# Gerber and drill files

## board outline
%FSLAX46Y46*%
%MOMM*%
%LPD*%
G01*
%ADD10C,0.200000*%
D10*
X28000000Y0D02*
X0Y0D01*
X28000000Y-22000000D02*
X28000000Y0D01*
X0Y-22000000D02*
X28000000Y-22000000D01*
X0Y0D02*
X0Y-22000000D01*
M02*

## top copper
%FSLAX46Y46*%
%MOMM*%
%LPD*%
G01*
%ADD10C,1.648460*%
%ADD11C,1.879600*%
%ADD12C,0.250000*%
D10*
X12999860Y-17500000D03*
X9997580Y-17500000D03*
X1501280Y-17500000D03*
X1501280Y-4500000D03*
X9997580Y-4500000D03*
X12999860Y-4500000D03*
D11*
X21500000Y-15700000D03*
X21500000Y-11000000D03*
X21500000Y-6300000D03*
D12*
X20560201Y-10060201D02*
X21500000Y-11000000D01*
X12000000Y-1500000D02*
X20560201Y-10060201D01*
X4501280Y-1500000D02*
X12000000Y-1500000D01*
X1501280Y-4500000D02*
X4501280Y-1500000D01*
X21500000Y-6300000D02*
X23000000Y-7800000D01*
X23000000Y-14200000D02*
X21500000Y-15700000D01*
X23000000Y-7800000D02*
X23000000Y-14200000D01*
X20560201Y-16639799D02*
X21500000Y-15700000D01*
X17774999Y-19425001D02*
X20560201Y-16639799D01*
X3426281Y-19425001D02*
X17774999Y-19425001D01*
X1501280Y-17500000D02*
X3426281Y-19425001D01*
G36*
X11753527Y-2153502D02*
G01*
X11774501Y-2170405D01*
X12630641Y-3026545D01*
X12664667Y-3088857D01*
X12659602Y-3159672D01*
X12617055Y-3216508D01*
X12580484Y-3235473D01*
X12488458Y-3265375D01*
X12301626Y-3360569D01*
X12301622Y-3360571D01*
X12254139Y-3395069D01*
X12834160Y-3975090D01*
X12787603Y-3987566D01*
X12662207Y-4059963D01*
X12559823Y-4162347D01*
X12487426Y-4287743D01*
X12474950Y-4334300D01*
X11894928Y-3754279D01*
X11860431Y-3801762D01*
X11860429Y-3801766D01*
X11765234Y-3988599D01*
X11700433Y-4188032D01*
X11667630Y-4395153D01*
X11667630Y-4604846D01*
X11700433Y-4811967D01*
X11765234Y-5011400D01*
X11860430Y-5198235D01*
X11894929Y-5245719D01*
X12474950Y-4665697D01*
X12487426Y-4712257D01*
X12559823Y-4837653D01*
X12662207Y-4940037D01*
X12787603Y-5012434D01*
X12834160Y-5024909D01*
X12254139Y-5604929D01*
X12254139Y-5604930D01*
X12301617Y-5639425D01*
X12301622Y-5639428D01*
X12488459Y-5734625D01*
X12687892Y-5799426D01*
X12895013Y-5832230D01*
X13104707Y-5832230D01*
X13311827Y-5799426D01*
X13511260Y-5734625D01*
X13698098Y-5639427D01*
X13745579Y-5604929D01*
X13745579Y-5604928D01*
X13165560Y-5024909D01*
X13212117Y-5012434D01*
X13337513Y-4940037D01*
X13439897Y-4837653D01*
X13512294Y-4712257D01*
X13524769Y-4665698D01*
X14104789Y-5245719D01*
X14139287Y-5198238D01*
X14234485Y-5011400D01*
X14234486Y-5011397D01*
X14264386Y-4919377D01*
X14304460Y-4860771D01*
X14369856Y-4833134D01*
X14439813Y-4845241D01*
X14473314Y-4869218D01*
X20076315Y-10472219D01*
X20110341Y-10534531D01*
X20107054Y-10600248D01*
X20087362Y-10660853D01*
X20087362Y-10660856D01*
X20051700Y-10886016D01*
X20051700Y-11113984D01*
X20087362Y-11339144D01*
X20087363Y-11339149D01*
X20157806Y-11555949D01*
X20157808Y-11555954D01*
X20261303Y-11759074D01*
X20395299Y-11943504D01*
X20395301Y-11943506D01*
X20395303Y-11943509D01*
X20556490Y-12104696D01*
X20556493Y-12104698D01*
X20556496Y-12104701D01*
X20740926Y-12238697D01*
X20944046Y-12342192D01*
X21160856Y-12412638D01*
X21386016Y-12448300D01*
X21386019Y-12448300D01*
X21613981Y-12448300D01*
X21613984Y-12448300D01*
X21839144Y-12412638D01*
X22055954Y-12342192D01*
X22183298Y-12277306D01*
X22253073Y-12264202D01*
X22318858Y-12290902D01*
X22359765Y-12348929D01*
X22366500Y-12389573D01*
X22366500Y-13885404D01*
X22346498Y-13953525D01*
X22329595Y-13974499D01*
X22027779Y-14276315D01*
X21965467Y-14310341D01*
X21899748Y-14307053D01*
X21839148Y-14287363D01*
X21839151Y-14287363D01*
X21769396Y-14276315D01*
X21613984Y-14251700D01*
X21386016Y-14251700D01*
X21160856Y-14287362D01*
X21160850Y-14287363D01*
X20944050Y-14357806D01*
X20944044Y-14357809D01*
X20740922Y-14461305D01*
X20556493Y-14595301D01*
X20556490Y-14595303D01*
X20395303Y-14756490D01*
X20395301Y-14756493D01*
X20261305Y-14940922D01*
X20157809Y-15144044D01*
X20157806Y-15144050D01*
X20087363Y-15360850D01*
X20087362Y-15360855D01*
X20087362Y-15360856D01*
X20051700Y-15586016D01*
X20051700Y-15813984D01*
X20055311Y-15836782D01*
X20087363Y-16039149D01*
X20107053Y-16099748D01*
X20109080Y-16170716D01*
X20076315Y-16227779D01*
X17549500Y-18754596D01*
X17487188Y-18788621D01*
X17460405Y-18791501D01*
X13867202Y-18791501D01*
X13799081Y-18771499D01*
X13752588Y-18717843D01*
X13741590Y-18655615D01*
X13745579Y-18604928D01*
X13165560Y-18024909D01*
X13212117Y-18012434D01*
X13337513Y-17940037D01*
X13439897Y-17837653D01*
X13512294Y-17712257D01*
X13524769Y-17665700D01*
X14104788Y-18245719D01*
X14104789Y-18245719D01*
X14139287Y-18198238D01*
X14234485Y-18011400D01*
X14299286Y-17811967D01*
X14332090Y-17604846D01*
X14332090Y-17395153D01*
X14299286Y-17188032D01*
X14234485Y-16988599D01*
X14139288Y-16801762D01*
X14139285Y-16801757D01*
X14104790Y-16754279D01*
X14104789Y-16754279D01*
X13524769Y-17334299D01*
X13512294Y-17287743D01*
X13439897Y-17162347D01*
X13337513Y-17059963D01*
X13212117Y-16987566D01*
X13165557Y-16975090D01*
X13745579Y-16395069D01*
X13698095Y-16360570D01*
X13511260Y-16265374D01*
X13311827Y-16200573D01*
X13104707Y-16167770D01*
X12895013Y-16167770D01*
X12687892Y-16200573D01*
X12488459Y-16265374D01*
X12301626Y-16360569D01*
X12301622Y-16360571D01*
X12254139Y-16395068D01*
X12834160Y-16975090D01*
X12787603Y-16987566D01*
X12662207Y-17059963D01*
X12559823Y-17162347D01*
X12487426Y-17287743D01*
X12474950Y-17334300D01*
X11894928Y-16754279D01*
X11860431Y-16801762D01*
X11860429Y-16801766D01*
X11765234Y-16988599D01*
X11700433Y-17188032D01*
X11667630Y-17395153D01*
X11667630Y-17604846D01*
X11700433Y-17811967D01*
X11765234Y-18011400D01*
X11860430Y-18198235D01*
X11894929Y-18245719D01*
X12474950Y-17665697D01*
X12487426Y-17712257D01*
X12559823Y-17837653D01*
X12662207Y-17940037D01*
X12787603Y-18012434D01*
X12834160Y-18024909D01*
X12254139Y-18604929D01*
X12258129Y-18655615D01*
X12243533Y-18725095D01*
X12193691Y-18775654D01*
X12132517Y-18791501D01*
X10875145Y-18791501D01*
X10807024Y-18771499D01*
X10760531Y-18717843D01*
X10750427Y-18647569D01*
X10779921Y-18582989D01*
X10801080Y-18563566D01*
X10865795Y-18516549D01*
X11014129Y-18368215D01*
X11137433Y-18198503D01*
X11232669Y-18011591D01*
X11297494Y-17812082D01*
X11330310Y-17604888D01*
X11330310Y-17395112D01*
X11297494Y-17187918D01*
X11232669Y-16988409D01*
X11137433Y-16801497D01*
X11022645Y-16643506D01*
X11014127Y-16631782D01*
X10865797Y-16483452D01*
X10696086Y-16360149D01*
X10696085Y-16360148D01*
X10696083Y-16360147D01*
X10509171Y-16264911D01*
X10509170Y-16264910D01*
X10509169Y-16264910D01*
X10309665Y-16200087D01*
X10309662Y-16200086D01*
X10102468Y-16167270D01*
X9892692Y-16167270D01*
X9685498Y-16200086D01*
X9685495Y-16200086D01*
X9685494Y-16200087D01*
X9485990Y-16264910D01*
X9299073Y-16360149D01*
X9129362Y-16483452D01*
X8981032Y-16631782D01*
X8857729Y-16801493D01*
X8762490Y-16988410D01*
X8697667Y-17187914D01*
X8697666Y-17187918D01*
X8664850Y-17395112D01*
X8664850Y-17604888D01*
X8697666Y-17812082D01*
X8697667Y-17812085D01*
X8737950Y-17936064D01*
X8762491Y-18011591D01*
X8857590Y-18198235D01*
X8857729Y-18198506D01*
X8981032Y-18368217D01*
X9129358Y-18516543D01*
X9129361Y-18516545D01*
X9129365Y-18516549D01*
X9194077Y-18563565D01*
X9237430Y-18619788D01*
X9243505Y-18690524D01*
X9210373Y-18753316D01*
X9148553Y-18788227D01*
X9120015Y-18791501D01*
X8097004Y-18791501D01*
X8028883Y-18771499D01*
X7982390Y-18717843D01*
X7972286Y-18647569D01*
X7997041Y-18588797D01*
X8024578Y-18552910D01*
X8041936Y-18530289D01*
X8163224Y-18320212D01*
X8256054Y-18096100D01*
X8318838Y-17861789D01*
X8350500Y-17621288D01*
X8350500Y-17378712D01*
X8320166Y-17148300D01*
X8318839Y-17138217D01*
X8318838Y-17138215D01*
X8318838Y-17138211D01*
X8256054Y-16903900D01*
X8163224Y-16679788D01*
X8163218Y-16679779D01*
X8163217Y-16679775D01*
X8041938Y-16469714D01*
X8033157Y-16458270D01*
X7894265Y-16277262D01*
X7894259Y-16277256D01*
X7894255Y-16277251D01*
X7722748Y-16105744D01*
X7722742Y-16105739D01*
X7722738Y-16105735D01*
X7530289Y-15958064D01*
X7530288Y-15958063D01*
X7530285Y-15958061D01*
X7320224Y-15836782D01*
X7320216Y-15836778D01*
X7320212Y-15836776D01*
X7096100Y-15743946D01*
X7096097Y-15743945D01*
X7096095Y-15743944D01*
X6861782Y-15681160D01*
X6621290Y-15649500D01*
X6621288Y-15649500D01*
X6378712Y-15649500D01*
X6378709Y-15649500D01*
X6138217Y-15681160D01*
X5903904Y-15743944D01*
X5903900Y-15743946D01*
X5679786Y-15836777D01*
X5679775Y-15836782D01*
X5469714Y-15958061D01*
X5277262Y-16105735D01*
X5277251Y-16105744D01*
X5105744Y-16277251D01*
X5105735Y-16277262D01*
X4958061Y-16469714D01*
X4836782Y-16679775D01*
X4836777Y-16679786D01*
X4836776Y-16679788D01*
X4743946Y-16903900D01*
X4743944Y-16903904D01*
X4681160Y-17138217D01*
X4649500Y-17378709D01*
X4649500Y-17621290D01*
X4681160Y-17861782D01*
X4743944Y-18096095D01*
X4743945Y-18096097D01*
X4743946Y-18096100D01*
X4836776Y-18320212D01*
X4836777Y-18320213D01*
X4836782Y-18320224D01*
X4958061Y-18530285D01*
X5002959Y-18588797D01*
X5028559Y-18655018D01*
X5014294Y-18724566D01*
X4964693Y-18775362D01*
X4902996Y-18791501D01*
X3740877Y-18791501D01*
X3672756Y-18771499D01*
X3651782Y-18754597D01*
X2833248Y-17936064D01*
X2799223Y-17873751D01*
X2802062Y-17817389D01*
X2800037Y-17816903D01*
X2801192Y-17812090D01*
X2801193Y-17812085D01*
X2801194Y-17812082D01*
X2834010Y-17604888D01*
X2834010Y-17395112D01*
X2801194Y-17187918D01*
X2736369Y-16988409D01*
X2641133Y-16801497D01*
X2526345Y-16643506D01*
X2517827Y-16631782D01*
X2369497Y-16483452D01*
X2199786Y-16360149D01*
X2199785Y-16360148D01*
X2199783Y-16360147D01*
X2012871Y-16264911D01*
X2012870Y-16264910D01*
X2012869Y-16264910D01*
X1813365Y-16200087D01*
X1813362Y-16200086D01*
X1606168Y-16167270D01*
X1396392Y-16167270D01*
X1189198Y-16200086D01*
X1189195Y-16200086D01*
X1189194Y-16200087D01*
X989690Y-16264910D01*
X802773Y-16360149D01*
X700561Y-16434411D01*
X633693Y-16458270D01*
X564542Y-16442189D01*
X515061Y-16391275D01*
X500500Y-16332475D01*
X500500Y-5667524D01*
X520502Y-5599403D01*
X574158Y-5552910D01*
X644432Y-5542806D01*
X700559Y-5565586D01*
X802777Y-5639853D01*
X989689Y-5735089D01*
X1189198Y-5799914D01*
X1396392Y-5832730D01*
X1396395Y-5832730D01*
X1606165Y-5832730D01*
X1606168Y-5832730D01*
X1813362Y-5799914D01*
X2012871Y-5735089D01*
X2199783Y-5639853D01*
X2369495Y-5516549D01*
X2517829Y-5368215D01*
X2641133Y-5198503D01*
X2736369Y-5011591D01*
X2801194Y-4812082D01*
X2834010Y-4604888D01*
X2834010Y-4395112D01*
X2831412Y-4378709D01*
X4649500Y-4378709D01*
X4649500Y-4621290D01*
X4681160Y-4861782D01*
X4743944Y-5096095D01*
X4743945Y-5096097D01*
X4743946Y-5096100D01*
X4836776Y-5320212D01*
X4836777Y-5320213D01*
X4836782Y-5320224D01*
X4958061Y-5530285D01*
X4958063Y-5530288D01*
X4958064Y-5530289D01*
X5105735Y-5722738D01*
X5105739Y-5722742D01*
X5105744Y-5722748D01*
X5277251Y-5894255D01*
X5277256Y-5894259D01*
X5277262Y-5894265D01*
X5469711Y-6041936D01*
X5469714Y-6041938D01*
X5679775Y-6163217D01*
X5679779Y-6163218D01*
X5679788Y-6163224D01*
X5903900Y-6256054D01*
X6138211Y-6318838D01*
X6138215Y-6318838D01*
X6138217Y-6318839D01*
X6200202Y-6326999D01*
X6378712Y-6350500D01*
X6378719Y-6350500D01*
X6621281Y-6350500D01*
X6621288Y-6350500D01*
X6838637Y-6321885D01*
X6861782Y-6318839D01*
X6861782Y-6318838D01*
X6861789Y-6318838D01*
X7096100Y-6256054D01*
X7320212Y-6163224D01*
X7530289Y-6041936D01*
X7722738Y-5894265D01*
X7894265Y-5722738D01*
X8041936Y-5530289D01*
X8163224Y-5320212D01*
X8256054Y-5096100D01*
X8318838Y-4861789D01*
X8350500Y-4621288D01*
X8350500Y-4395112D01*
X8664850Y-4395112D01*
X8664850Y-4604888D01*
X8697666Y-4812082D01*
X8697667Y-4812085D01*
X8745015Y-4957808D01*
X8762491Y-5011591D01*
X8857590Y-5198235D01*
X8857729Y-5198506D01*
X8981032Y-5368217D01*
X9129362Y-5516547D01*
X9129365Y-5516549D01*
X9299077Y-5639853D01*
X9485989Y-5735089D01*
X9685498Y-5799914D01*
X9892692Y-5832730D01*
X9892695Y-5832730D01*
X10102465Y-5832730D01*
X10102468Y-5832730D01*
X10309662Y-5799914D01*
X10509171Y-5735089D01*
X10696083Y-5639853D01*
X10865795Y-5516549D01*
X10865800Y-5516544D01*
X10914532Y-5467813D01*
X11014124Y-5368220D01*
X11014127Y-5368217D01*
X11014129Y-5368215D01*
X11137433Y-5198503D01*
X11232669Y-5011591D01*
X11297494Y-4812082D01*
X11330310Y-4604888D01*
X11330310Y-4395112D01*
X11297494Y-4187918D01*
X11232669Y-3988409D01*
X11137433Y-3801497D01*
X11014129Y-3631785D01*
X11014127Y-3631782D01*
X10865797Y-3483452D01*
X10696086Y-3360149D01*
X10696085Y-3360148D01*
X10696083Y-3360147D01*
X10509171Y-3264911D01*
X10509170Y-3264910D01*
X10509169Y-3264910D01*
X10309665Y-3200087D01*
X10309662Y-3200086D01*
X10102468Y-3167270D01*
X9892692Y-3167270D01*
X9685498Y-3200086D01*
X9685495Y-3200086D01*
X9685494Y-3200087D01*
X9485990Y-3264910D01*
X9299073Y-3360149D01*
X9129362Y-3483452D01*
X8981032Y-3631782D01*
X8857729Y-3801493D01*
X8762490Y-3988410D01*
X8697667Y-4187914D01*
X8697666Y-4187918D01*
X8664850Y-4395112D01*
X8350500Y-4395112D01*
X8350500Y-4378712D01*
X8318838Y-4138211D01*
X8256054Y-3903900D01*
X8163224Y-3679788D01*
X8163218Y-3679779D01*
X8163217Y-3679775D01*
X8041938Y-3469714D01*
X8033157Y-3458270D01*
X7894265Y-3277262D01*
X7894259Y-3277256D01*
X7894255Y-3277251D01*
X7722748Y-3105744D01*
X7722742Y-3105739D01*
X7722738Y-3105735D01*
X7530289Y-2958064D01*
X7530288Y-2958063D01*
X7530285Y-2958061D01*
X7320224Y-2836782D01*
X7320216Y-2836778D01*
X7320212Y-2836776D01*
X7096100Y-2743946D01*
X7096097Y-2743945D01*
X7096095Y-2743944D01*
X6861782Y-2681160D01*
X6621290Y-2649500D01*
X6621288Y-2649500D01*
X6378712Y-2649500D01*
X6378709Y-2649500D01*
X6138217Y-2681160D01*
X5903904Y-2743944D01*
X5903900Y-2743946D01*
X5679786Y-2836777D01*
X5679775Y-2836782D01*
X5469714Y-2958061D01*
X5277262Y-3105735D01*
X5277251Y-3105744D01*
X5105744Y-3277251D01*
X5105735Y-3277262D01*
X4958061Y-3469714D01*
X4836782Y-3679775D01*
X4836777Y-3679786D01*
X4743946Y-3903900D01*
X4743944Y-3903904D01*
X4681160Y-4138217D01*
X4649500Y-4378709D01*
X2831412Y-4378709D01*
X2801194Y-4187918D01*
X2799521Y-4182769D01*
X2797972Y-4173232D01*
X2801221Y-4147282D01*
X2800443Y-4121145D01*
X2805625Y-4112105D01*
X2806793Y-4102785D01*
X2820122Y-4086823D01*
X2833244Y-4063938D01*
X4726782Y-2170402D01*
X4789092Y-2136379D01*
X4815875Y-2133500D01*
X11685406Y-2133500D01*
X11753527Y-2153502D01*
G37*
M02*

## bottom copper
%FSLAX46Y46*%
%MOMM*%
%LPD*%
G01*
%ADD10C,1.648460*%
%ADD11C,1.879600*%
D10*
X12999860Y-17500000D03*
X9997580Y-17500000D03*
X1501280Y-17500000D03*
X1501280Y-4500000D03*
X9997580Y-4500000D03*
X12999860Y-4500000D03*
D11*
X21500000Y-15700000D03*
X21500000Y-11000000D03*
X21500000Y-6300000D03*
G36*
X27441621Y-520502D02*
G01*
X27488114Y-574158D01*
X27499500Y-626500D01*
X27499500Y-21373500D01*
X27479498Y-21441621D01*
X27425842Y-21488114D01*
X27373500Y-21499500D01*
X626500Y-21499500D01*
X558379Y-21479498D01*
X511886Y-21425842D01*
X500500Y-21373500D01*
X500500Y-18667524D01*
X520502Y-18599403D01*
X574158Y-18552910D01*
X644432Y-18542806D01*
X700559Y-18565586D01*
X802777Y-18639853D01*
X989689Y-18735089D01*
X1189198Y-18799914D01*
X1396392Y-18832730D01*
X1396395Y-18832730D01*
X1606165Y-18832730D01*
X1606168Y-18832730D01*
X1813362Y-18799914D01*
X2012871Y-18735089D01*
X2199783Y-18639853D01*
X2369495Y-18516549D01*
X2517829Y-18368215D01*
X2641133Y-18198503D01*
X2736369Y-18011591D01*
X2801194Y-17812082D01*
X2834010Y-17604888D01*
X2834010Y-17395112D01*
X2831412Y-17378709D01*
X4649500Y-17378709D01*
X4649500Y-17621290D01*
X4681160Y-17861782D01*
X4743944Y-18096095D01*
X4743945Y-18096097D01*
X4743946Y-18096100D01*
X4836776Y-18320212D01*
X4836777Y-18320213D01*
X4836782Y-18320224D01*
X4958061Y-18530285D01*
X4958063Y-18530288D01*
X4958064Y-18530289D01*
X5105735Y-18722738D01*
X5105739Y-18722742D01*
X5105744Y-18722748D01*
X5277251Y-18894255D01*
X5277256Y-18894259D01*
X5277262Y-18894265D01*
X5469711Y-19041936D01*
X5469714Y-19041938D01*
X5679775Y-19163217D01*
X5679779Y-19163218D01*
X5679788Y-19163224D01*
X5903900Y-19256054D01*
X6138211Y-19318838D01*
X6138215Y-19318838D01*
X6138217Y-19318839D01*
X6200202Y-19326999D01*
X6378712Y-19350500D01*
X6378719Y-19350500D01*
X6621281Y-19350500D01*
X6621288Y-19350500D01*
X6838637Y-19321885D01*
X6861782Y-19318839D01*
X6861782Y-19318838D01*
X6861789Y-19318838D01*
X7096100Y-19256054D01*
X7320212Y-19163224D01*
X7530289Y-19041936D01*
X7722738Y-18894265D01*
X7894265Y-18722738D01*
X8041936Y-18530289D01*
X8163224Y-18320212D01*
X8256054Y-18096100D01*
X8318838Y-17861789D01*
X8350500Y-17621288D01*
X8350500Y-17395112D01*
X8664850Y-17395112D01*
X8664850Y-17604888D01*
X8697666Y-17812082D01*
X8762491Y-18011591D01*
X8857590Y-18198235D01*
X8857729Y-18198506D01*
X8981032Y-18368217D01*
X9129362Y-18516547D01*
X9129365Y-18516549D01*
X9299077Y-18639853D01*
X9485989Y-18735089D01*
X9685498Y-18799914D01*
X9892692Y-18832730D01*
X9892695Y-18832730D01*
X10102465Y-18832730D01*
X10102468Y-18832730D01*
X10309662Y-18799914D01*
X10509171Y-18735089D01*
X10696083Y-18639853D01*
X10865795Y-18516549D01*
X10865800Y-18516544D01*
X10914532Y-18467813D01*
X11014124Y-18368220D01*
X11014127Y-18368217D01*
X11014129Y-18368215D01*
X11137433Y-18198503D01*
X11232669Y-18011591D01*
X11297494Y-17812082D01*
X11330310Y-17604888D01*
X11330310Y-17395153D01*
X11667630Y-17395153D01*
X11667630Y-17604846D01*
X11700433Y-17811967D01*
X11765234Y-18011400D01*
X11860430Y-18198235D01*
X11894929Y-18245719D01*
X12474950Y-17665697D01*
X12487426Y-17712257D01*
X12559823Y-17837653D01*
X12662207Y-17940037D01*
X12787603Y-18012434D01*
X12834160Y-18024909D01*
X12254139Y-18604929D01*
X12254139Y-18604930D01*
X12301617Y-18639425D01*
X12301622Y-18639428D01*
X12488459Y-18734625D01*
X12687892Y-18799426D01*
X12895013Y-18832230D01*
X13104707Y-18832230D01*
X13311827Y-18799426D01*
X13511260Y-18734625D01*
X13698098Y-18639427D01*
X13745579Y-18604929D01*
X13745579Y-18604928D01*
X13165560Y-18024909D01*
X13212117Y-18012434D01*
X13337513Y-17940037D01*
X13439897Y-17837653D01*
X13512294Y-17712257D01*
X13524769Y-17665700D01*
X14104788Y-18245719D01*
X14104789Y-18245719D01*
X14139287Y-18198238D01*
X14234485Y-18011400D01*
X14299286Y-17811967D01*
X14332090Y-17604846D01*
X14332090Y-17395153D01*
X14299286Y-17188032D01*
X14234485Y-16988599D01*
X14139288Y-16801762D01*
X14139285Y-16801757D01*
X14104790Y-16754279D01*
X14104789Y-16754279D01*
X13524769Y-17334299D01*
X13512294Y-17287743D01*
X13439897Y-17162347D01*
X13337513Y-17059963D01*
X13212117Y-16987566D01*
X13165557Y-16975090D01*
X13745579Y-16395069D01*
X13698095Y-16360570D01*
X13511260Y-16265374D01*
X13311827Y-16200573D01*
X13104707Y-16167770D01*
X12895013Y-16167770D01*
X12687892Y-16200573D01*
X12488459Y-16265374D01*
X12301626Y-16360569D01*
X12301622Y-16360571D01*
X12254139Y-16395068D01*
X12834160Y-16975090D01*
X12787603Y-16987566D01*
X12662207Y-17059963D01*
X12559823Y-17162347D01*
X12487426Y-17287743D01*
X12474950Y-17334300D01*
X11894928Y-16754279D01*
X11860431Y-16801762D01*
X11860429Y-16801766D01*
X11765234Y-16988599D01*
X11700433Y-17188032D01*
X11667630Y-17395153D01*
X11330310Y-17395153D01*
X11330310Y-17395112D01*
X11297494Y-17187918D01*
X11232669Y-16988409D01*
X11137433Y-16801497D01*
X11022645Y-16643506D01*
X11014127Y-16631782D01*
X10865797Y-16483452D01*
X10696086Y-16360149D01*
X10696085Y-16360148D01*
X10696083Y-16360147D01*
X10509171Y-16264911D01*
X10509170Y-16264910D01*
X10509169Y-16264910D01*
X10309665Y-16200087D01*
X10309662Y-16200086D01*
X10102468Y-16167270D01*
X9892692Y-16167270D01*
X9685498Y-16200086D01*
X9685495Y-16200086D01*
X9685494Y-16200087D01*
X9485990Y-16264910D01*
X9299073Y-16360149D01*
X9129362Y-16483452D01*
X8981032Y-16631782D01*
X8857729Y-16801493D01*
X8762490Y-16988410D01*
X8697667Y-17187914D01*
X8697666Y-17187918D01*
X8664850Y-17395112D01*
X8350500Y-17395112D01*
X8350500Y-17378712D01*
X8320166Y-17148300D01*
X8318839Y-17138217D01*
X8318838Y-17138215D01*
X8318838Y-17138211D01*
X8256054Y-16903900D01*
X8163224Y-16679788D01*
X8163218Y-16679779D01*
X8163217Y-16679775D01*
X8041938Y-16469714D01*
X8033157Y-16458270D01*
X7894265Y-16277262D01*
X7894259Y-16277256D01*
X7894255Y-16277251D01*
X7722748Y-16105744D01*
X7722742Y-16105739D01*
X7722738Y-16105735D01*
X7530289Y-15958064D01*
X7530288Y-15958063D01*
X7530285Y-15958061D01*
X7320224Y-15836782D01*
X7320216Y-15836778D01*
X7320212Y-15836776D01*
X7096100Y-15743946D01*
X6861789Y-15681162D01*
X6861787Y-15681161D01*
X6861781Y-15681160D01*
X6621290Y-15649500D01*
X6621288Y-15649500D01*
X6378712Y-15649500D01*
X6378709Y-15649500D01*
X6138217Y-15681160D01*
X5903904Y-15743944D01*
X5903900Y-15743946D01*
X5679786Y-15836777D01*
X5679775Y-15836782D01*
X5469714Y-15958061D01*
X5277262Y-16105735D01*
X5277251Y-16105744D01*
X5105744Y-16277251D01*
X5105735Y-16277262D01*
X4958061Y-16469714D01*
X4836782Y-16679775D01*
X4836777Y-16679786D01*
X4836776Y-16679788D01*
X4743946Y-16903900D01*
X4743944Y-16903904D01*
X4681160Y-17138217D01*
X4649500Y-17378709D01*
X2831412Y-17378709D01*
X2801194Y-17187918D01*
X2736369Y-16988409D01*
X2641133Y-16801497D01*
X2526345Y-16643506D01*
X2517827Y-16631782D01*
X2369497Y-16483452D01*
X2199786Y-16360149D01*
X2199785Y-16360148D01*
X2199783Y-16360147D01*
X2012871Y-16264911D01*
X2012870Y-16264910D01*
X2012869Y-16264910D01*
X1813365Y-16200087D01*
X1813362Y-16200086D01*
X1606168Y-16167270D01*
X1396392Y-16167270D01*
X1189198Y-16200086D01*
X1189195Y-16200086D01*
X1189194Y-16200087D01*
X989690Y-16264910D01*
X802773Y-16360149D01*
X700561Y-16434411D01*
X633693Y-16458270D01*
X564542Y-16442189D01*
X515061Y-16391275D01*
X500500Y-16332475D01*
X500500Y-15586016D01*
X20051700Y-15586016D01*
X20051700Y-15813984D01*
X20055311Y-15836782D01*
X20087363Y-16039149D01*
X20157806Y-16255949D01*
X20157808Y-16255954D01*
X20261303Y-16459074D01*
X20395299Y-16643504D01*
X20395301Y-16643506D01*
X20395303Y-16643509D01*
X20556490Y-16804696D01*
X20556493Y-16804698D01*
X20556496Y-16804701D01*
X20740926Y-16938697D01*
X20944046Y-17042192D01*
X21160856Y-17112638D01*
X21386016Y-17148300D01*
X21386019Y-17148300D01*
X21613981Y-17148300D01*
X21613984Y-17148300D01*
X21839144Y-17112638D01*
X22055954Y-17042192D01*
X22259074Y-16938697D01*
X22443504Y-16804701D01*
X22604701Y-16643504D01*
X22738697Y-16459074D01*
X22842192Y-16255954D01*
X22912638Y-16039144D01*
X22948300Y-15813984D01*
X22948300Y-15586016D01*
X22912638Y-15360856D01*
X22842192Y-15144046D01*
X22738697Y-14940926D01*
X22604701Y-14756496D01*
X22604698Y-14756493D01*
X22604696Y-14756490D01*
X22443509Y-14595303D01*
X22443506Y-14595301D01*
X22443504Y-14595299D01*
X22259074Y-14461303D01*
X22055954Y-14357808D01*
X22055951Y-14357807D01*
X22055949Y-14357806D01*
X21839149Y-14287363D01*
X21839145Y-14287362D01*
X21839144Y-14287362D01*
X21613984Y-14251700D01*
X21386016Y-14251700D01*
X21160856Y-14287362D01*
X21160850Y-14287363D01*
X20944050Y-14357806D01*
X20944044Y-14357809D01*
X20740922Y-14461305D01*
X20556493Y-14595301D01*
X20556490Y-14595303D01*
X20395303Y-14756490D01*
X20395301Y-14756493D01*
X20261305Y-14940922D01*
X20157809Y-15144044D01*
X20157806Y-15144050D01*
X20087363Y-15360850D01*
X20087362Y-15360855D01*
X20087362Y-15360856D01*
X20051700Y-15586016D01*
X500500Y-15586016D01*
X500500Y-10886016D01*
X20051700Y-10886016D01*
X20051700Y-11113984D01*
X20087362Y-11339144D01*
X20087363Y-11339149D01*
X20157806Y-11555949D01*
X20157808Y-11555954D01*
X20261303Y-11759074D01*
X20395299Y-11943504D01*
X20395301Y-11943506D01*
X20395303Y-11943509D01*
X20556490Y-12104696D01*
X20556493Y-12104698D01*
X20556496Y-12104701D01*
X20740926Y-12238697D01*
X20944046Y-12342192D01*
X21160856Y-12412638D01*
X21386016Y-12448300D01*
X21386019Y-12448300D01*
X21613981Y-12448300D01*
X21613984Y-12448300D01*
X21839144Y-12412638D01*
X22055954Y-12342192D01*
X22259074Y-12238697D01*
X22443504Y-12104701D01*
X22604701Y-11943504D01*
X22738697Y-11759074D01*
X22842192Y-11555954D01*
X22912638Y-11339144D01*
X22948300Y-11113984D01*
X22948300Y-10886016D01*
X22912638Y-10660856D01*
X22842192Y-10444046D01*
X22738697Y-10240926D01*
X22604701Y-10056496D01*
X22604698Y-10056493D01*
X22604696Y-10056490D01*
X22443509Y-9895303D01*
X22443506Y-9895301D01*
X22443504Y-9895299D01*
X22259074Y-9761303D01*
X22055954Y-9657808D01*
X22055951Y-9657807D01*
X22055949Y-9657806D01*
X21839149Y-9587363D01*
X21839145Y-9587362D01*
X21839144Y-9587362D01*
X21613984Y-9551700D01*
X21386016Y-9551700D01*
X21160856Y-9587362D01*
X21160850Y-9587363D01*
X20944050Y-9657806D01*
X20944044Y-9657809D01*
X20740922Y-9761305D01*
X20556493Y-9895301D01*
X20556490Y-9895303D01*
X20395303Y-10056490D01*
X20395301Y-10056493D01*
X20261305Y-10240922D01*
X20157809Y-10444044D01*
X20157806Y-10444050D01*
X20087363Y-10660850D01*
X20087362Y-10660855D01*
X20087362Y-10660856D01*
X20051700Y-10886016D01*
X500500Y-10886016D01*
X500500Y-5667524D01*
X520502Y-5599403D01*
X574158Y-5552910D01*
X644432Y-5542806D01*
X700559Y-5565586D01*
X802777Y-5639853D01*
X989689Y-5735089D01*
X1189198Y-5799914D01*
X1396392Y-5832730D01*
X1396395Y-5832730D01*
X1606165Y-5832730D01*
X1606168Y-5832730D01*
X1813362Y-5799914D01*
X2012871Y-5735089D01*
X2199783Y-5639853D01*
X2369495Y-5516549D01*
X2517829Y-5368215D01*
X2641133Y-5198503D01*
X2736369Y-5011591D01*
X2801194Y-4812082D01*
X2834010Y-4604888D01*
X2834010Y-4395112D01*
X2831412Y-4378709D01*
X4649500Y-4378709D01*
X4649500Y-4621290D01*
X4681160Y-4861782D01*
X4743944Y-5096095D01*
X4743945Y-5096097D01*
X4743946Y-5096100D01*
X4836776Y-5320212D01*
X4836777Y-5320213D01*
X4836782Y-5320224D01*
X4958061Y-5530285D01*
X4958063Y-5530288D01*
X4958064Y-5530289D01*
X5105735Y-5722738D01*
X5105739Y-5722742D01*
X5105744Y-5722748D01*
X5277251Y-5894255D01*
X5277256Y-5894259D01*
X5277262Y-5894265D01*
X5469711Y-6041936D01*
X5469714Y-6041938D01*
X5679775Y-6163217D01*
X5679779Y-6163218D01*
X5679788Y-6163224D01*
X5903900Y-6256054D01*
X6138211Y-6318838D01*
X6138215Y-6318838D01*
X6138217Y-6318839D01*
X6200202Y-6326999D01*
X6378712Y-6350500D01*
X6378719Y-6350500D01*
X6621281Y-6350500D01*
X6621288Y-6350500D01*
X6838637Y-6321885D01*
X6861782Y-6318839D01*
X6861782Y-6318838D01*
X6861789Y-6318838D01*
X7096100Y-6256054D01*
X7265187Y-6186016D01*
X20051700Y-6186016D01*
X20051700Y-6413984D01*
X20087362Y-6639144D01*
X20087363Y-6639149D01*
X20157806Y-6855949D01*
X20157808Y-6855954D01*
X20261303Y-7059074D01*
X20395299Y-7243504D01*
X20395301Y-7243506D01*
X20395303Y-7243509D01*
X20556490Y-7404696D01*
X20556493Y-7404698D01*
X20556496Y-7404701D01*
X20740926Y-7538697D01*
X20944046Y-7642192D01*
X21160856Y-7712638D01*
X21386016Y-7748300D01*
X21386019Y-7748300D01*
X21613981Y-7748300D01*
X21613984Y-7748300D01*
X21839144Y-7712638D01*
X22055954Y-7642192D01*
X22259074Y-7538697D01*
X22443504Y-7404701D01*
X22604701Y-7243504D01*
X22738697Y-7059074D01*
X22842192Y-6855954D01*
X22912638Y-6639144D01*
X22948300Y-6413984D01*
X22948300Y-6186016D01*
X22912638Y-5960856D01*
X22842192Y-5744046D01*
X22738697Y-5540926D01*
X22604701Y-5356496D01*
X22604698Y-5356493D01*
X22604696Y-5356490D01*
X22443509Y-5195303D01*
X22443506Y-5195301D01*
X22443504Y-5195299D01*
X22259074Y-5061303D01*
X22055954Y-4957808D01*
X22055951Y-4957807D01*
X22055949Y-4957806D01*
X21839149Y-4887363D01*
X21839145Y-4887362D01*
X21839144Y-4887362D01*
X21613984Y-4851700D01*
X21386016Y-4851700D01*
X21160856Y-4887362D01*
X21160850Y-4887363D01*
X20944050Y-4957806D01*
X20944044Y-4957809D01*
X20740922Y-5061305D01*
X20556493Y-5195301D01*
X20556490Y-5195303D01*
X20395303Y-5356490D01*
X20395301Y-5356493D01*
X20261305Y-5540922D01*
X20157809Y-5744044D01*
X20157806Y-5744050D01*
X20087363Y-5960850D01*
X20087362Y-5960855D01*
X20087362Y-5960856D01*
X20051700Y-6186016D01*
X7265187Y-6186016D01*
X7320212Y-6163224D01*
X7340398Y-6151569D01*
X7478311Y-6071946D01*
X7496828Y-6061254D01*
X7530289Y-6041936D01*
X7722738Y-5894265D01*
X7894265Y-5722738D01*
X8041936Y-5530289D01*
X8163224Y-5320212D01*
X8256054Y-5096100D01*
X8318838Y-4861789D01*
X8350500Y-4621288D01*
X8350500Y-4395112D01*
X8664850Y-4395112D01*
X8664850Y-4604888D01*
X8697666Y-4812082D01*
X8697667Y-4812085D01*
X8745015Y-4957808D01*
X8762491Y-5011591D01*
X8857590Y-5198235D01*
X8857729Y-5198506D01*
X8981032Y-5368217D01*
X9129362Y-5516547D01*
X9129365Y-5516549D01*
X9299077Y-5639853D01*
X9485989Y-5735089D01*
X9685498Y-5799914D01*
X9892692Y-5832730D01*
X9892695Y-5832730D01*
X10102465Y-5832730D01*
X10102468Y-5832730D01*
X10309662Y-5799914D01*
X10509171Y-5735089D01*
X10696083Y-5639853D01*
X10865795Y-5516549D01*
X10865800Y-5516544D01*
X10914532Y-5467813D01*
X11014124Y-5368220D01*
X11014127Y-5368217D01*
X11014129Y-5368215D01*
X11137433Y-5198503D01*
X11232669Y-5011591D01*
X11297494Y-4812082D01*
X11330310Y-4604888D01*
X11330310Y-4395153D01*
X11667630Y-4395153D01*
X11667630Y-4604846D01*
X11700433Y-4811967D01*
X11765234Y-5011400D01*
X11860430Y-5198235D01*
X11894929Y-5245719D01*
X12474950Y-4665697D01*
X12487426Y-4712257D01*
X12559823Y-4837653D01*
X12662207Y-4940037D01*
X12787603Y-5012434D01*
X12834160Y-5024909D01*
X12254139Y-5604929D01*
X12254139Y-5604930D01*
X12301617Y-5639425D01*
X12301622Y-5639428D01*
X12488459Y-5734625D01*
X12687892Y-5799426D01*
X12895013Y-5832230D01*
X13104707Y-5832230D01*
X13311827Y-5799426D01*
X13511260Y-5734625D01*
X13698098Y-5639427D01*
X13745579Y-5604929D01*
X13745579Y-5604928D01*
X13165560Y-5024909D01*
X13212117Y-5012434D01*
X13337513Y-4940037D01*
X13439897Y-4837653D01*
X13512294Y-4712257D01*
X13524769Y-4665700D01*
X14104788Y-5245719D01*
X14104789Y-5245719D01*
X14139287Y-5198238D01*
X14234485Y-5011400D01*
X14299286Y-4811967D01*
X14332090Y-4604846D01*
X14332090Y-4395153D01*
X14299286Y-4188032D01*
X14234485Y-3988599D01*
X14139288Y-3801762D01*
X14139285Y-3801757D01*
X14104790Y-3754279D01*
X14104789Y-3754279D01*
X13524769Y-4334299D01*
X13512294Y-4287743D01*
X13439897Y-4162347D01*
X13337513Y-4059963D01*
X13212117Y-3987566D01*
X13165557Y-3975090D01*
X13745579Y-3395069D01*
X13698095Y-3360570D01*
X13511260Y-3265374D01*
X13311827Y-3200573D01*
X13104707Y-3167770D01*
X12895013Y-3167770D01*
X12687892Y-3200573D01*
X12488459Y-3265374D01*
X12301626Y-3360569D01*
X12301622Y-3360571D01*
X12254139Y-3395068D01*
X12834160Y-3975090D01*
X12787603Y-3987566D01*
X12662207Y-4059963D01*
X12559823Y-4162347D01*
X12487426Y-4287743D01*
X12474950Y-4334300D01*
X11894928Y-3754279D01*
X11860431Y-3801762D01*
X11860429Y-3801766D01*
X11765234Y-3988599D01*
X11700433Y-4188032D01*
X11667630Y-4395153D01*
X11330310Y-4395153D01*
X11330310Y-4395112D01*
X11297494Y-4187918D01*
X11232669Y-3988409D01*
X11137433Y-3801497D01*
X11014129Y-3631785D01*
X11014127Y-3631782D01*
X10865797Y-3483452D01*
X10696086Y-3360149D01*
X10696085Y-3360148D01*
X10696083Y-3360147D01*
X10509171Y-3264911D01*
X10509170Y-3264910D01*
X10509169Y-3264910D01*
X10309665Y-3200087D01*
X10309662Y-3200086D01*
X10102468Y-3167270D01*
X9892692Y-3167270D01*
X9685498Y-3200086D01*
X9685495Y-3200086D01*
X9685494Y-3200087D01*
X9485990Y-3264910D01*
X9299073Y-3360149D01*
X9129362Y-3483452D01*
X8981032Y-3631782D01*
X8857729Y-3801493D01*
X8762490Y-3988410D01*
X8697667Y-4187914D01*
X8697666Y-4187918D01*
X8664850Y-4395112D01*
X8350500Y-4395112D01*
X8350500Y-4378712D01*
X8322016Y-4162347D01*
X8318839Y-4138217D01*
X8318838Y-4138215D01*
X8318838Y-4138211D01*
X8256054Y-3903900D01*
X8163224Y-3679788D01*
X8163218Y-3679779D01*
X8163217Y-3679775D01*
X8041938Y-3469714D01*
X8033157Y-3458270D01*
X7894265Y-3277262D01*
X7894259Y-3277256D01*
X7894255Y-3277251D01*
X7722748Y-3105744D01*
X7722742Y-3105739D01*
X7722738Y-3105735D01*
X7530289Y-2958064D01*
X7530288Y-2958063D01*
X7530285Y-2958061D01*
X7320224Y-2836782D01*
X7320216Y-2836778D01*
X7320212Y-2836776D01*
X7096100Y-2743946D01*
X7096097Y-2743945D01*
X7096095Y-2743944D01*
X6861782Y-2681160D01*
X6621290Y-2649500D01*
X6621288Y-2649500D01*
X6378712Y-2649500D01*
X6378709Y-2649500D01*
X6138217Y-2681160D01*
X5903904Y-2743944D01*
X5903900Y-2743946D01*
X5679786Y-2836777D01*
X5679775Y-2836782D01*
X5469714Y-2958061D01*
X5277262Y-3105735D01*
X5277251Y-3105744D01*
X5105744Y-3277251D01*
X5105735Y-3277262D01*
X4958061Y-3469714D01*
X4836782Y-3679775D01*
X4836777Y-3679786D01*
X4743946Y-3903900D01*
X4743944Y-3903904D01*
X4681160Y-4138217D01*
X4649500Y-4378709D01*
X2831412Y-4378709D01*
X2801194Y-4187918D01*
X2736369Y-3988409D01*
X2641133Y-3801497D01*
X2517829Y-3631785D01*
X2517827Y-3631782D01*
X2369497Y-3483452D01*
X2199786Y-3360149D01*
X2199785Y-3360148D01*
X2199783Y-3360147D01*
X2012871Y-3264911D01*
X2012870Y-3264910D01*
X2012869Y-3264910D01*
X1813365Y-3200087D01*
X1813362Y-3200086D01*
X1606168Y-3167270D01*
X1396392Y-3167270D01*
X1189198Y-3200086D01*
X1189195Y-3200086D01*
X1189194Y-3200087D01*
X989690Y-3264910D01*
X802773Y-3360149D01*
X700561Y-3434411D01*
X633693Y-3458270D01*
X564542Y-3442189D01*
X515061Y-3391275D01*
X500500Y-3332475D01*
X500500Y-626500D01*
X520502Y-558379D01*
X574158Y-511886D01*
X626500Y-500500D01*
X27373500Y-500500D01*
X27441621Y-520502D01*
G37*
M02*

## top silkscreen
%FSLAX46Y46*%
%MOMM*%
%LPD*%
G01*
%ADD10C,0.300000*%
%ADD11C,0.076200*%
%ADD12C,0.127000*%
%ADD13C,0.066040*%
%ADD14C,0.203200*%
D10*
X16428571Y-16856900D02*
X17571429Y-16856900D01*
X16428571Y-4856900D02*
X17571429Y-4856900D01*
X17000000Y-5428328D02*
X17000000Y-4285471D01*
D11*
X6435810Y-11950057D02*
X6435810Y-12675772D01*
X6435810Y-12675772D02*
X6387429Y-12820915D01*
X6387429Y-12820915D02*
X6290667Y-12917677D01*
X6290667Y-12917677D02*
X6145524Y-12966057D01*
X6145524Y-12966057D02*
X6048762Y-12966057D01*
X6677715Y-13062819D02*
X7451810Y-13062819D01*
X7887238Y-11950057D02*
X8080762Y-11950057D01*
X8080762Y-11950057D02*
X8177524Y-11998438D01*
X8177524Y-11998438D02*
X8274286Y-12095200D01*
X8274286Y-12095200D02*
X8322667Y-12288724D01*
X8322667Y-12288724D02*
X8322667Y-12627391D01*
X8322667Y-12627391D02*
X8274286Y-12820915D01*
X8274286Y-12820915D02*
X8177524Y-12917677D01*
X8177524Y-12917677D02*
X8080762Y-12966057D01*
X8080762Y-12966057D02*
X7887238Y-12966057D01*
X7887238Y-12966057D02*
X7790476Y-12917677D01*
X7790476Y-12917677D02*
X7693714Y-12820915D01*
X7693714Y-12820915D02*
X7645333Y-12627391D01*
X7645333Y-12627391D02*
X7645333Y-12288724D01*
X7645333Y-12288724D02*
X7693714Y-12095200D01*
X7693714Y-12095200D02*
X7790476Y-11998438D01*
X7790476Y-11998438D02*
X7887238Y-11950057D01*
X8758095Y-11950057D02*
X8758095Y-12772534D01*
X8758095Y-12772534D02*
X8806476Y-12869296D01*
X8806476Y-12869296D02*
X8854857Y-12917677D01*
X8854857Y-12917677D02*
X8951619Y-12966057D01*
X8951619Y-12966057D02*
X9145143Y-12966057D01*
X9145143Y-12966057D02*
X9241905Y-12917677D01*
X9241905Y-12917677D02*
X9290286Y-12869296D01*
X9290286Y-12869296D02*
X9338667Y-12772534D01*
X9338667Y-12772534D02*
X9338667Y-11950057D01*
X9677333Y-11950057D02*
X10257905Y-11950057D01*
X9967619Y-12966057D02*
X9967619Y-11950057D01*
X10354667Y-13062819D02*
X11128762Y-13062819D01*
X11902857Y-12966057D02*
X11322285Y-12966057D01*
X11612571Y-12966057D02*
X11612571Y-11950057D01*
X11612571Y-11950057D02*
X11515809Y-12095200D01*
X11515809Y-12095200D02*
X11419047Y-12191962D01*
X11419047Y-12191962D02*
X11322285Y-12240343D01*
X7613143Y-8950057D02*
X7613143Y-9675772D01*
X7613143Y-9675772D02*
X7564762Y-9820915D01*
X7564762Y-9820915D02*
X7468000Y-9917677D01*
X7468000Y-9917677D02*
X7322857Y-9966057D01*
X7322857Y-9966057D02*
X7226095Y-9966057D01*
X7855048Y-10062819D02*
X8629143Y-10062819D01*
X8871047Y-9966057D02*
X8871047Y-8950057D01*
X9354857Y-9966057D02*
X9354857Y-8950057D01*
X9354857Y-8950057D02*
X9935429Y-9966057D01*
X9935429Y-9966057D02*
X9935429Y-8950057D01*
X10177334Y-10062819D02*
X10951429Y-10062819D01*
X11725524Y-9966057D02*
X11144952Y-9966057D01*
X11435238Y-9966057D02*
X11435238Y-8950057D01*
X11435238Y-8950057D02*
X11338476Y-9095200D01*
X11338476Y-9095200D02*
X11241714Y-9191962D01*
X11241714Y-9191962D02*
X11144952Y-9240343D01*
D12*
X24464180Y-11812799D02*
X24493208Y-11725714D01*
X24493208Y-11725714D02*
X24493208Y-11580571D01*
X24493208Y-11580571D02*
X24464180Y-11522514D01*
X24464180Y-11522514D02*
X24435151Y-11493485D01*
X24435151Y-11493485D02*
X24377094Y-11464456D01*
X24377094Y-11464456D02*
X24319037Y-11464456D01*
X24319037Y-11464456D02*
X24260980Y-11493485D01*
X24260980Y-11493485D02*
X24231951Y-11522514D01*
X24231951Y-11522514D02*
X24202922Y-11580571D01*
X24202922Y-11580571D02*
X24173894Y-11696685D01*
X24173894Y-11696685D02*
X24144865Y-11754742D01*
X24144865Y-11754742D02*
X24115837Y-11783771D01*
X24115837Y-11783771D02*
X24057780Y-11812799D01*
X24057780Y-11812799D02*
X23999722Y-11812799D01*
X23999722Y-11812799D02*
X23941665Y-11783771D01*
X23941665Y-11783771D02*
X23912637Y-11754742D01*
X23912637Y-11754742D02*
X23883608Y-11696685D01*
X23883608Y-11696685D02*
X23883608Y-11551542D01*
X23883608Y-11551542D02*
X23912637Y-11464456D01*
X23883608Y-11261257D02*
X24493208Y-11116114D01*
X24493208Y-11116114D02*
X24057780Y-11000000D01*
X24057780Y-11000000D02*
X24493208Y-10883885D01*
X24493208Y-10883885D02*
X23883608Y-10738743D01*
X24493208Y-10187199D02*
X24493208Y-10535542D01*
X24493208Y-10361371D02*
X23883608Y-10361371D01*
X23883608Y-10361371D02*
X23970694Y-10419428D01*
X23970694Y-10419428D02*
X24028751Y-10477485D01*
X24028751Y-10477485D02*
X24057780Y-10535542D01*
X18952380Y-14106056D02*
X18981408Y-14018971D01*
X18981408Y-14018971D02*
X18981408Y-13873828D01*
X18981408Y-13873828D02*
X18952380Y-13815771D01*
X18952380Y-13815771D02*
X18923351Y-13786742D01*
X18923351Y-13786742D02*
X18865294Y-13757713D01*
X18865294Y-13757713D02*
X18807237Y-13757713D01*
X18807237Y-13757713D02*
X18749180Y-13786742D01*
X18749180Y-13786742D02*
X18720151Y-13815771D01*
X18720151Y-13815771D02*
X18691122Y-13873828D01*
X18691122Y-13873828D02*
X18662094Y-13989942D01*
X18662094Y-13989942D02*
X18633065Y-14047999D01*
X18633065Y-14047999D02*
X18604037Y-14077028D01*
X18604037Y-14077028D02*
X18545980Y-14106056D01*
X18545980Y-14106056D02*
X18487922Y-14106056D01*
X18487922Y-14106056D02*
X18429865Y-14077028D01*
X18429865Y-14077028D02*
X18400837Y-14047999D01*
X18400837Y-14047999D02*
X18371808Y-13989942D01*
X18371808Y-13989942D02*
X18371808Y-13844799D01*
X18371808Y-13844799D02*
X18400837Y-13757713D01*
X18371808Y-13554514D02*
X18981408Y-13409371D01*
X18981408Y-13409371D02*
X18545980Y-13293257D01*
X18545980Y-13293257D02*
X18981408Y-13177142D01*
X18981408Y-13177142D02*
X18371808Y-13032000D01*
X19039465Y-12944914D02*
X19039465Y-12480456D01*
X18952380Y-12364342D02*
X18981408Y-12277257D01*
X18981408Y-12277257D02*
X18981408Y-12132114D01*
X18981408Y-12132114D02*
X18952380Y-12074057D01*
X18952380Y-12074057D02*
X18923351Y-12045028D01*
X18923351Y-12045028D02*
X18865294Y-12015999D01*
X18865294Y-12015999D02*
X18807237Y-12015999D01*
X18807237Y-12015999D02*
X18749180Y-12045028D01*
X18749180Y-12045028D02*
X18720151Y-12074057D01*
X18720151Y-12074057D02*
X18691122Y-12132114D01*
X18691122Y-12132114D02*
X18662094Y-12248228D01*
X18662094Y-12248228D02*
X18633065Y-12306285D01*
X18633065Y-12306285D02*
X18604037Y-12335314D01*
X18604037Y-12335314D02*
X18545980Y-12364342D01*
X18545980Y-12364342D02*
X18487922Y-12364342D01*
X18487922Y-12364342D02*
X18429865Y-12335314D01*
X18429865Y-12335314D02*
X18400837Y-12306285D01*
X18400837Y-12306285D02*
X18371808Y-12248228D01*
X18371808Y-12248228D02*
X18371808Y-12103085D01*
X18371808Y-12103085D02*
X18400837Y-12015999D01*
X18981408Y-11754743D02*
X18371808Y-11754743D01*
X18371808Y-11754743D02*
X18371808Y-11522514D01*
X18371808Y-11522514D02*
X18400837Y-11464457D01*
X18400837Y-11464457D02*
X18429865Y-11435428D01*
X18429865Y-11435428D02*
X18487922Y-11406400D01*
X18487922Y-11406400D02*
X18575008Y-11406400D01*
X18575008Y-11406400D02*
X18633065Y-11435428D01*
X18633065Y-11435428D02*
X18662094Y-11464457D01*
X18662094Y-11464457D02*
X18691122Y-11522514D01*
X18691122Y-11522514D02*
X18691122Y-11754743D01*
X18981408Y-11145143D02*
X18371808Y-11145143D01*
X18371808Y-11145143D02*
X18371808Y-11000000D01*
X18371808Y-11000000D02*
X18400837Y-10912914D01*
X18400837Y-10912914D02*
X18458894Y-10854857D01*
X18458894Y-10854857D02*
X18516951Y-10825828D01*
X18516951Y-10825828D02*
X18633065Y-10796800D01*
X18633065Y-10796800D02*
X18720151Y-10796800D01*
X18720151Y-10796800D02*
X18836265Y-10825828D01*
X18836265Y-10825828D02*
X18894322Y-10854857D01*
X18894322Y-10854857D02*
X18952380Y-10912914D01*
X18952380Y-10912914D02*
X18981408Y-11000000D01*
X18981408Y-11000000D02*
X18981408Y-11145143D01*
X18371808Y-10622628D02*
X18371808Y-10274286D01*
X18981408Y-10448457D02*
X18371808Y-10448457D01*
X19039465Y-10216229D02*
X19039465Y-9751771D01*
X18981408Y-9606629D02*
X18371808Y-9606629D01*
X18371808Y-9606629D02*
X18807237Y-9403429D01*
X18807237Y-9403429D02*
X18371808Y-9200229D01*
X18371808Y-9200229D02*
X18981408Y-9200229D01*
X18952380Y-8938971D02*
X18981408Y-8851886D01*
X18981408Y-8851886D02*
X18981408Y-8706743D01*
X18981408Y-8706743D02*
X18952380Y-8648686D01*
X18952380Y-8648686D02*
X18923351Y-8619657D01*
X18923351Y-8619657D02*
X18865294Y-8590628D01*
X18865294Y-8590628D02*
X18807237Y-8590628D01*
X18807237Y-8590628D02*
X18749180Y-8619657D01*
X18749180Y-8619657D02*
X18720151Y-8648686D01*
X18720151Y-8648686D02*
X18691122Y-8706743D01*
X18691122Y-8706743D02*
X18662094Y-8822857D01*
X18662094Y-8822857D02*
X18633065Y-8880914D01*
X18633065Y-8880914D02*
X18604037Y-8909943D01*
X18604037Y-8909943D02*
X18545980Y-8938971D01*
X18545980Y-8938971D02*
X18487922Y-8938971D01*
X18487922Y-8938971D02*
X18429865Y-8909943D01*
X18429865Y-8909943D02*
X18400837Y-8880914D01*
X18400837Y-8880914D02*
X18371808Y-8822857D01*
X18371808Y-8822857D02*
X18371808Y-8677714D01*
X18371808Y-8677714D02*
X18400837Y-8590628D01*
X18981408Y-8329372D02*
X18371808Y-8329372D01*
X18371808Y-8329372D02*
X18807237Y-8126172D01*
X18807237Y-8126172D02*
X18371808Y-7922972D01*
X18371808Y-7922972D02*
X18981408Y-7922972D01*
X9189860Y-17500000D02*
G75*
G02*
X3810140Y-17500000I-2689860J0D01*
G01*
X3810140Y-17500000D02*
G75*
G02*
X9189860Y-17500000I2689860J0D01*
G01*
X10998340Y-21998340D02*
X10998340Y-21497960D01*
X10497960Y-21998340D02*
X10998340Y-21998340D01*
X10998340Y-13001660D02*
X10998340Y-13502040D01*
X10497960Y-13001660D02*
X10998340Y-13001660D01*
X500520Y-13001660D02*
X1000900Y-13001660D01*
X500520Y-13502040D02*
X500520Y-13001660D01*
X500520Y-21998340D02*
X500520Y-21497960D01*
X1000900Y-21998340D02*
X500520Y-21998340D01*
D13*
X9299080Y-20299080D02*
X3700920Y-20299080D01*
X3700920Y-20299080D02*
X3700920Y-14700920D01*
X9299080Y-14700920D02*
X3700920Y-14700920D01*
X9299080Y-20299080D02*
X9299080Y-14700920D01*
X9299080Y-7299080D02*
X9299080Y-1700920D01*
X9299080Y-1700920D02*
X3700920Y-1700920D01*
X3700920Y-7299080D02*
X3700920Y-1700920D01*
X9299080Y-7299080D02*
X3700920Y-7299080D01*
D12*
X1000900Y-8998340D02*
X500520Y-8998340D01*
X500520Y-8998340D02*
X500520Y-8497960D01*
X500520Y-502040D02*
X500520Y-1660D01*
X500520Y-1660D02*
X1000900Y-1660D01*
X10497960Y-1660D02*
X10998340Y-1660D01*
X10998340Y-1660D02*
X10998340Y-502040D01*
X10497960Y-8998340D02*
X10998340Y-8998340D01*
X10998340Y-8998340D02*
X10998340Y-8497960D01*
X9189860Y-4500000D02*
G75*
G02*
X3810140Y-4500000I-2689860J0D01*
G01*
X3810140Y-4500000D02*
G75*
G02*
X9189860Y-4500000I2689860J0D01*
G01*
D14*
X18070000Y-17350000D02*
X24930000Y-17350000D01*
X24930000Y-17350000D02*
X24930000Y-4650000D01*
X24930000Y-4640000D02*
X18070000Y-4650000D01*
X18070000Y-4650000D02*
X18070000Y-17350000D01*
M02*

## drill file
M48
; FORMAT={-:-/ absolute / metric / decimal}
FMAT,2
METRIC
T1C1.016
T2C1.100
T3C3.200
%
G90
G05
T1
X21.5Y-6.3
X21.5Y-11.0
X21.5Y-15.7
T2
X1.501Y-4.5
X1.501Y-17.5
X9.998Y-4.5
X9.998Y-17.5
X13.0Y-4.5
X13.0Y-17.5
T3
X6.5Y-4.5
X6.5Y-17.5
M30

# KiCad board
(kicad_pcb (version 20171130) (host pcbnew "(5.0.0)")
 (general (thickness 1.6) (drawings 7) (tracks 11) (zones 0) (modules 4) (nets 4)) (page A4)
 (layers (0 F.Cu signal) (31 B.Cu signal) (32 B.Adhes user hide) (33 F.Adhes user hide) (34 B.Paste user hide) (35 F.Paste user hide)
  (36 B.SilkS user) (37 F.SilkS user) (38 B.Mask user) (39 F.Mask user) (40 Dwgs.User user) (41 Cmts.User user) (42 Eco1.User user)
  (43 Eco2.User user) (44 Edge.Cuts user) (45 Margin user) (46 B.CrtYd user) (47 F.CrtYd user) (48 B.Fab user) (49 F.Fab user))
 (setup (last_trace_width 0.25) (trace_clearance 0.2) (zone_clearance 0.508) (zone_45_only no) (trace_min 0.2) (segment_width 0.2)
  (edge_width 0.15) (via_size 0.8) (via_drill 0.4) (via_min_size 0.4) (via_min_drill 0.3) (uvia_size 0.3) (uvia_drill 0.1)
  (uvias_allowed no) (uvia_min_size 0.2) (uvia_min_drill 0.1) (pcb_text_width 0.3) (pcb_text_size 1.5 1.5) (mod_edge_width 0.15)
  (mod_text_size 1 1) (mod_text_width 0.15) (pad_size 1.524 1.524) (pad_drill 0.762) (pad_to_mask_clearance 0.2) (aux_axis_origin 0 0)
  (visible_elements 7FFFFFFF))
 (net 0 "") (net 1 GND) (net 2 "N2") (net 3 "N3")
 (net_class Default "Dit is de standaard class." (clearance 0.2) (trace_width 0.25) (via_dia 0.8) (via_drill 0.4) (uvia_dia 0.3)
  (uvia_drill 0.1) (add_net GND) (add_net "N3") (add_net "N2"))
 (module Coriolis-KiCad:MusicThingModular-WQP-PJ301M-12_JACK (layer F.Cu) (at 6.5 17.5 90)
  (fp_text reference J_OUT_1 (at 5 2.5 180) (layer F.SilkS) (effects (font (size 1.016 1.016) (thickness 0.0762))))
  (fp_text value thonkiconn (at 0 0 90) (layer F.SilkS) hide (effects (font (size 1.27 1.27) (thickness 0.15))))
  (fp_circle (center 0 0) (end 0 -2.68986) (layer F.SilkS) (width 0.127))
  (fp_line (start -4.49834 4.49834) (end -3.99796 4.49834) (layer F.SilkS) (width 0.127))
  (fp_line (start -4.49834 3.99796) (end -4.49834 4.49834) (layer F.SilkS) (width 0.127))
  (fp_line (start 4.49834 4.49834) (end 3.99796 4.49834) (layer F.SilkS) (width 0.127))
  (fp_line (start 4.49834 3.99796) (end 4.49834 4.49834) (layer F.SilkS) (width 0.127))
  (fp_line (start 4.49834 -5.99948) (end 4.49834 -5.4991) (layer F.SilkS) (width 0.127))
  (fp_line (start 3.99796 -5.99948) (end 4.49834 -5.99948) (layer F.SilkS) (width 0.127))
  (fp_line (start -4.49834 -5.99948) (end -3.99796 -5.99948) (layer F.SilkS) (width 0.127))
  (fp_line (start -4.49834 -5.4991) (end -4.49834 -5.99948) (layer F.SilkS) (width 0.127))
  (fp_line (start -2.79908 2.79908) (end -2.79908 -2.79908) (layer F.SilkS) (width 0.06604))
  (fp_line (start -2.79908 -2.79908) (end 2.79908 -2.79908) (layer F.SilkS) (width 0.06604))
  (fp_line (start 2.79908 2.79908) (end 2.79908 -2.79908) (layer F.SilkS) (width 0.06604))
  (fp_line (start -2.79908 2.79908) (end 2.79908 2.79908) (layer F.SilkS) (width 0.06604))
  (pad "" np_thru_hole circle (at 0 0 90) (size 3.2 3.2) (drill 3.2) (layers *.Cu *.Mask))
  (pad P$3_SLEEVE thru_hole circle (at 0 6.49986 90) (size 1.64846 1.64846) (drill 1.09982) (layers *.Cu *.Paste *.Mask) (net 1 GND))
  (pad P$2_SWITCH thru_hole circle (at 0 3.49758 90) (size 1.64846 1.64846) (drill 1.09982) (layers *.Cu *.Paste *.Mask))
  (pad P$1_TIP thru_hole circle (at 0 -4.99872 90) (size 1.64846 1.64846) (drill 1.09982) (layers *.Cu *.Paste *.Mask) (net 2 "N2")))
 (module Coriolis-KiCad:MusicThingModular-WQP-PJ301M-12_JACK (layer F.Cu) (at 6.5 4.5 90)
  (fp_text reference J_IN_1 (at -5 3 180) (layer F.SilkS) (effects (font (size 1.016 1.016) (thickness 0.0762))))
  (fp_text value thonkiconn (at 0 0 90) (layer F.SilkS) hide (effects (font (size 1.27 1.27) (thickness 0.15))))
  (fp_line (start -2.79908 2.79908) (end 2.79908 2.79908) (layer F.SilkS) (width 0.06604))
  (fp_line (start 2.79908 2.79908) (end 2.79908 -2.79908) (layer F.SilkS) (width 0.06604))
  (fp_line (start -2.79908 -2.79908) (end 2.79908 -2.79908) (layer F.SilkS) (width 0.06604))
  (fp_line (start -2.79908 2.79908) (end -2.79908 -2.79908) (layer F.SilkS) (width 0.06604))
  (fp_line (start -4.49834 -5.4991) (end -4.49834 -5.99948) (layer F.SilkS) (width 0.127))
  (fp_line (start -4.49834 -5.99948) (end -3.99796 -5.99948) (layer F.SilkS) (width 0.127))
  (fp_line (start 3.99796 -5.99948) (end 4.49834 -5.99948) (layer F.SilkS) (width 0.127))
  (fp_line (start 4.49834 -5.99948) (end 4.49834 -5.4991) (layer F.SilkS) (width 0.127))
  (fp_line (start 4.49834 3.99796) (end 4.49834 4.49834) (layer F.SilkS) (width 0.127))
  (fp_line (start 4.49834 4.49834) (end 3.99796 4.49834) (layer F.SilkS) (width 0.127))
  (fp_line (start -4.49834 3.99796) (end -4.49834 4.49834) (layer F.SilkS) (width 0.127))
  (fp_line (start -4.49834 4.49834) (end -3.99796 4.49834) (layer F.SilkS) (width 0.127))
  (fp_circle (center 0 0) (end 0 -2.68986) (layer F.SilkS) (width 0.127))
  (pad P$1_TIP thru_hole circle (at 0 -4.99872 90) (size 1.64846 1.64846) (drill 1.09982) (layers *.Cu *.Paste *.Mask) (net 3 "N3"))
  (pad P$2_SWITCH thru_hole circle (at 0 3.49758 90) (size 1.64846 1.64846) (drill 1.09982) (layers *.Cu *.Paste *.Mask))
  (pad P$3_SLEEVE thru_hole circle (at 0 6.49986 90) (size 1.64846 1.64846) (drill 1.09982) (layers *.Cu *.Paste *.Mask) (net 1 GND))
  (pad "" np_thru_hole circle (at 0 0 90) (size 3.2 3.2) (drill 3.2) (layers *.Cu *.Mask)))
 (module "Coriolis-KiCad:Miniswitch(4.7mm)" (layer F.Cu) (at 21.5 11 180)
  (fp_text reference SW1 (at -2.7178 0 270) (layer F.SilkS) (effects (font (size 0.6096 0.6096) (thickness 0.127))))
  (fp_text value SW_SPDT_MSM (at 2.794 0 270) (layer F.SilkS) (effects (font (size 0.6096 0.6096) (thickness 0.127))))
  (fp_line (start 3.43 -6.35) (end -3.43 -6.35) (layer F.SilkS) (width 0.2032))
  (fp_line (start -3.43 -6.35) (end -3.43 6.35) (layer F.SilkS) (width 0.2032))
  (fp_line (start -3.43 6.36) (end 3.43 6.35) (layer F.SilkS) (width 0.2032))
  (fp_line (start 3.43 6.35) (end 3.43 -6.35) (layer F.SilkS) (width 0.2032))
  (pad 1 thru_hole circle (at 0 -4.7 180) (size 1.8796 1.8796) (drill 1.016) (layers *.Cu *.Mask) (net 2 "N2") (solder_mask_margin 0.1016))
  (pad 2 thru_hole circle (at 0 0 180) (size 1.8796 1.8796) (drill 1.016) (layers *.Cu *.Mask) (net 3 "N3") (solder_mask_margin 0.1016))
  (pad 3 thru_hole circle (at 0 4.7 180) (size 1.8796 1.8796) (drill 1.016) (layers *.Cu *.Mask) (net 2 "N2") (solder_mask_margin 0.1016)))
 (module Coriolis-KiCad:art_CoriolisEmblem (layer B.Cu) (at 1.5 20)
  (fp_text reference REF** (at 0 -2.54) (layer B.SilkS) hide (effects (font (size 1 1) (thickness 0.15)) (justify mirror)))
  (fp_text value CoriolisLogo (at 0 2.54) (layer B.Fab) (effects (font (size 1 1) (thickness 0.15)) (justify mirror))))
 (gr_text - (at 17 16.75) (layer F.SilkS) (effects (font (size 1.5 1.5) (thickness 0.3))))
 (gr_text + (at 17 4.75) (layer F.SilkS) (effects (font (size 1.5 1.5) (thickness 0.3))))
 (gr_line (start 28 0) (end 0 0) (layer Edge.Cuts) (width 0.2))
 (gr_line (start 28 22) (end 28 0) (layer Edge.Cuts) (width 0.2))
 (gr_line (start 0 22) (end 28 22) (layer Edge.Cuts) (width 0.2))
 (gr_line (start 0 0) (end 0 22) (layer Edge.Cuts) (width 0.2))
 (segment (start 20.560201 10.060201) (end 21.5 11) (width 0.25) (layer F.Cu) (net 3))
 (segment (start 12 1.5) (end 20.560201 10.060201) (width 0.25) (layer F.Cu) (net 3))
 (segment (start 4.50128 1.5) (end 12 1.5) (width 0.25) (layer F.Cu) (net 3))
 (segment (start 1.50128 4.5) (end 4.50128 1.5) (width 0.25) (layer F.Cu) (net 3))
 (segment (start 21.5 6.3) (end 23 7.8) (width 0.25) (layer F.Cu) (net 2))
 (segment (start 23 14.2) (end 21.5 15.7) (width 0.25) (layer F.Cu) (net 2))
 (segment (start 23 7.8) (end 23 14.2) (width 0.25) (layer F.Cu) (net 2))
 (segment (start 20.560201 16.639799) (end 21.5 15.7) (width 0.25) (layer F.Cu) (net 2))
 (segment (start 17.774999 19.425001) (end 20.560201 16.639799) (width 0.25) (layer F.Cu) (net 2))
 (segment (start 3.426281 19.425001) (end 17.774999 19.425001) (width 0.25) (layer F.Cu) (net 2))
 (segment (start 1.50128 17.5) (end 3.426281 19.425001) (width 0.25) (layer F.Cu) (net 2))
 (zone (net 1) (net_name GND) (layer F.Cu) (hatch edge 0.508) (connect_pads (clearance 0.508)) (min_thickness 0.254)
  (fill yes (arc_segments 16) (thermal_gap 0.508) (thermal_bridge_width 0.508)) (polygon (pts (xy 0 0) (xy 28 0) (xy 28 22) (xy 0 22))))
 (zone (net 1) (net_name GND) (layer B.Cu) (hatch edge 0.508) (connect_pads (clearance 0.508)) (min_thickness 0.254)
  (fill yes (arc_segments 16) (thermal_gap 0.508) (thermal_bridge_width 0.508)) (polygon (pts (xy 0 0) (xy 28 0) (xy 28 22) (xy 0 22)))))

